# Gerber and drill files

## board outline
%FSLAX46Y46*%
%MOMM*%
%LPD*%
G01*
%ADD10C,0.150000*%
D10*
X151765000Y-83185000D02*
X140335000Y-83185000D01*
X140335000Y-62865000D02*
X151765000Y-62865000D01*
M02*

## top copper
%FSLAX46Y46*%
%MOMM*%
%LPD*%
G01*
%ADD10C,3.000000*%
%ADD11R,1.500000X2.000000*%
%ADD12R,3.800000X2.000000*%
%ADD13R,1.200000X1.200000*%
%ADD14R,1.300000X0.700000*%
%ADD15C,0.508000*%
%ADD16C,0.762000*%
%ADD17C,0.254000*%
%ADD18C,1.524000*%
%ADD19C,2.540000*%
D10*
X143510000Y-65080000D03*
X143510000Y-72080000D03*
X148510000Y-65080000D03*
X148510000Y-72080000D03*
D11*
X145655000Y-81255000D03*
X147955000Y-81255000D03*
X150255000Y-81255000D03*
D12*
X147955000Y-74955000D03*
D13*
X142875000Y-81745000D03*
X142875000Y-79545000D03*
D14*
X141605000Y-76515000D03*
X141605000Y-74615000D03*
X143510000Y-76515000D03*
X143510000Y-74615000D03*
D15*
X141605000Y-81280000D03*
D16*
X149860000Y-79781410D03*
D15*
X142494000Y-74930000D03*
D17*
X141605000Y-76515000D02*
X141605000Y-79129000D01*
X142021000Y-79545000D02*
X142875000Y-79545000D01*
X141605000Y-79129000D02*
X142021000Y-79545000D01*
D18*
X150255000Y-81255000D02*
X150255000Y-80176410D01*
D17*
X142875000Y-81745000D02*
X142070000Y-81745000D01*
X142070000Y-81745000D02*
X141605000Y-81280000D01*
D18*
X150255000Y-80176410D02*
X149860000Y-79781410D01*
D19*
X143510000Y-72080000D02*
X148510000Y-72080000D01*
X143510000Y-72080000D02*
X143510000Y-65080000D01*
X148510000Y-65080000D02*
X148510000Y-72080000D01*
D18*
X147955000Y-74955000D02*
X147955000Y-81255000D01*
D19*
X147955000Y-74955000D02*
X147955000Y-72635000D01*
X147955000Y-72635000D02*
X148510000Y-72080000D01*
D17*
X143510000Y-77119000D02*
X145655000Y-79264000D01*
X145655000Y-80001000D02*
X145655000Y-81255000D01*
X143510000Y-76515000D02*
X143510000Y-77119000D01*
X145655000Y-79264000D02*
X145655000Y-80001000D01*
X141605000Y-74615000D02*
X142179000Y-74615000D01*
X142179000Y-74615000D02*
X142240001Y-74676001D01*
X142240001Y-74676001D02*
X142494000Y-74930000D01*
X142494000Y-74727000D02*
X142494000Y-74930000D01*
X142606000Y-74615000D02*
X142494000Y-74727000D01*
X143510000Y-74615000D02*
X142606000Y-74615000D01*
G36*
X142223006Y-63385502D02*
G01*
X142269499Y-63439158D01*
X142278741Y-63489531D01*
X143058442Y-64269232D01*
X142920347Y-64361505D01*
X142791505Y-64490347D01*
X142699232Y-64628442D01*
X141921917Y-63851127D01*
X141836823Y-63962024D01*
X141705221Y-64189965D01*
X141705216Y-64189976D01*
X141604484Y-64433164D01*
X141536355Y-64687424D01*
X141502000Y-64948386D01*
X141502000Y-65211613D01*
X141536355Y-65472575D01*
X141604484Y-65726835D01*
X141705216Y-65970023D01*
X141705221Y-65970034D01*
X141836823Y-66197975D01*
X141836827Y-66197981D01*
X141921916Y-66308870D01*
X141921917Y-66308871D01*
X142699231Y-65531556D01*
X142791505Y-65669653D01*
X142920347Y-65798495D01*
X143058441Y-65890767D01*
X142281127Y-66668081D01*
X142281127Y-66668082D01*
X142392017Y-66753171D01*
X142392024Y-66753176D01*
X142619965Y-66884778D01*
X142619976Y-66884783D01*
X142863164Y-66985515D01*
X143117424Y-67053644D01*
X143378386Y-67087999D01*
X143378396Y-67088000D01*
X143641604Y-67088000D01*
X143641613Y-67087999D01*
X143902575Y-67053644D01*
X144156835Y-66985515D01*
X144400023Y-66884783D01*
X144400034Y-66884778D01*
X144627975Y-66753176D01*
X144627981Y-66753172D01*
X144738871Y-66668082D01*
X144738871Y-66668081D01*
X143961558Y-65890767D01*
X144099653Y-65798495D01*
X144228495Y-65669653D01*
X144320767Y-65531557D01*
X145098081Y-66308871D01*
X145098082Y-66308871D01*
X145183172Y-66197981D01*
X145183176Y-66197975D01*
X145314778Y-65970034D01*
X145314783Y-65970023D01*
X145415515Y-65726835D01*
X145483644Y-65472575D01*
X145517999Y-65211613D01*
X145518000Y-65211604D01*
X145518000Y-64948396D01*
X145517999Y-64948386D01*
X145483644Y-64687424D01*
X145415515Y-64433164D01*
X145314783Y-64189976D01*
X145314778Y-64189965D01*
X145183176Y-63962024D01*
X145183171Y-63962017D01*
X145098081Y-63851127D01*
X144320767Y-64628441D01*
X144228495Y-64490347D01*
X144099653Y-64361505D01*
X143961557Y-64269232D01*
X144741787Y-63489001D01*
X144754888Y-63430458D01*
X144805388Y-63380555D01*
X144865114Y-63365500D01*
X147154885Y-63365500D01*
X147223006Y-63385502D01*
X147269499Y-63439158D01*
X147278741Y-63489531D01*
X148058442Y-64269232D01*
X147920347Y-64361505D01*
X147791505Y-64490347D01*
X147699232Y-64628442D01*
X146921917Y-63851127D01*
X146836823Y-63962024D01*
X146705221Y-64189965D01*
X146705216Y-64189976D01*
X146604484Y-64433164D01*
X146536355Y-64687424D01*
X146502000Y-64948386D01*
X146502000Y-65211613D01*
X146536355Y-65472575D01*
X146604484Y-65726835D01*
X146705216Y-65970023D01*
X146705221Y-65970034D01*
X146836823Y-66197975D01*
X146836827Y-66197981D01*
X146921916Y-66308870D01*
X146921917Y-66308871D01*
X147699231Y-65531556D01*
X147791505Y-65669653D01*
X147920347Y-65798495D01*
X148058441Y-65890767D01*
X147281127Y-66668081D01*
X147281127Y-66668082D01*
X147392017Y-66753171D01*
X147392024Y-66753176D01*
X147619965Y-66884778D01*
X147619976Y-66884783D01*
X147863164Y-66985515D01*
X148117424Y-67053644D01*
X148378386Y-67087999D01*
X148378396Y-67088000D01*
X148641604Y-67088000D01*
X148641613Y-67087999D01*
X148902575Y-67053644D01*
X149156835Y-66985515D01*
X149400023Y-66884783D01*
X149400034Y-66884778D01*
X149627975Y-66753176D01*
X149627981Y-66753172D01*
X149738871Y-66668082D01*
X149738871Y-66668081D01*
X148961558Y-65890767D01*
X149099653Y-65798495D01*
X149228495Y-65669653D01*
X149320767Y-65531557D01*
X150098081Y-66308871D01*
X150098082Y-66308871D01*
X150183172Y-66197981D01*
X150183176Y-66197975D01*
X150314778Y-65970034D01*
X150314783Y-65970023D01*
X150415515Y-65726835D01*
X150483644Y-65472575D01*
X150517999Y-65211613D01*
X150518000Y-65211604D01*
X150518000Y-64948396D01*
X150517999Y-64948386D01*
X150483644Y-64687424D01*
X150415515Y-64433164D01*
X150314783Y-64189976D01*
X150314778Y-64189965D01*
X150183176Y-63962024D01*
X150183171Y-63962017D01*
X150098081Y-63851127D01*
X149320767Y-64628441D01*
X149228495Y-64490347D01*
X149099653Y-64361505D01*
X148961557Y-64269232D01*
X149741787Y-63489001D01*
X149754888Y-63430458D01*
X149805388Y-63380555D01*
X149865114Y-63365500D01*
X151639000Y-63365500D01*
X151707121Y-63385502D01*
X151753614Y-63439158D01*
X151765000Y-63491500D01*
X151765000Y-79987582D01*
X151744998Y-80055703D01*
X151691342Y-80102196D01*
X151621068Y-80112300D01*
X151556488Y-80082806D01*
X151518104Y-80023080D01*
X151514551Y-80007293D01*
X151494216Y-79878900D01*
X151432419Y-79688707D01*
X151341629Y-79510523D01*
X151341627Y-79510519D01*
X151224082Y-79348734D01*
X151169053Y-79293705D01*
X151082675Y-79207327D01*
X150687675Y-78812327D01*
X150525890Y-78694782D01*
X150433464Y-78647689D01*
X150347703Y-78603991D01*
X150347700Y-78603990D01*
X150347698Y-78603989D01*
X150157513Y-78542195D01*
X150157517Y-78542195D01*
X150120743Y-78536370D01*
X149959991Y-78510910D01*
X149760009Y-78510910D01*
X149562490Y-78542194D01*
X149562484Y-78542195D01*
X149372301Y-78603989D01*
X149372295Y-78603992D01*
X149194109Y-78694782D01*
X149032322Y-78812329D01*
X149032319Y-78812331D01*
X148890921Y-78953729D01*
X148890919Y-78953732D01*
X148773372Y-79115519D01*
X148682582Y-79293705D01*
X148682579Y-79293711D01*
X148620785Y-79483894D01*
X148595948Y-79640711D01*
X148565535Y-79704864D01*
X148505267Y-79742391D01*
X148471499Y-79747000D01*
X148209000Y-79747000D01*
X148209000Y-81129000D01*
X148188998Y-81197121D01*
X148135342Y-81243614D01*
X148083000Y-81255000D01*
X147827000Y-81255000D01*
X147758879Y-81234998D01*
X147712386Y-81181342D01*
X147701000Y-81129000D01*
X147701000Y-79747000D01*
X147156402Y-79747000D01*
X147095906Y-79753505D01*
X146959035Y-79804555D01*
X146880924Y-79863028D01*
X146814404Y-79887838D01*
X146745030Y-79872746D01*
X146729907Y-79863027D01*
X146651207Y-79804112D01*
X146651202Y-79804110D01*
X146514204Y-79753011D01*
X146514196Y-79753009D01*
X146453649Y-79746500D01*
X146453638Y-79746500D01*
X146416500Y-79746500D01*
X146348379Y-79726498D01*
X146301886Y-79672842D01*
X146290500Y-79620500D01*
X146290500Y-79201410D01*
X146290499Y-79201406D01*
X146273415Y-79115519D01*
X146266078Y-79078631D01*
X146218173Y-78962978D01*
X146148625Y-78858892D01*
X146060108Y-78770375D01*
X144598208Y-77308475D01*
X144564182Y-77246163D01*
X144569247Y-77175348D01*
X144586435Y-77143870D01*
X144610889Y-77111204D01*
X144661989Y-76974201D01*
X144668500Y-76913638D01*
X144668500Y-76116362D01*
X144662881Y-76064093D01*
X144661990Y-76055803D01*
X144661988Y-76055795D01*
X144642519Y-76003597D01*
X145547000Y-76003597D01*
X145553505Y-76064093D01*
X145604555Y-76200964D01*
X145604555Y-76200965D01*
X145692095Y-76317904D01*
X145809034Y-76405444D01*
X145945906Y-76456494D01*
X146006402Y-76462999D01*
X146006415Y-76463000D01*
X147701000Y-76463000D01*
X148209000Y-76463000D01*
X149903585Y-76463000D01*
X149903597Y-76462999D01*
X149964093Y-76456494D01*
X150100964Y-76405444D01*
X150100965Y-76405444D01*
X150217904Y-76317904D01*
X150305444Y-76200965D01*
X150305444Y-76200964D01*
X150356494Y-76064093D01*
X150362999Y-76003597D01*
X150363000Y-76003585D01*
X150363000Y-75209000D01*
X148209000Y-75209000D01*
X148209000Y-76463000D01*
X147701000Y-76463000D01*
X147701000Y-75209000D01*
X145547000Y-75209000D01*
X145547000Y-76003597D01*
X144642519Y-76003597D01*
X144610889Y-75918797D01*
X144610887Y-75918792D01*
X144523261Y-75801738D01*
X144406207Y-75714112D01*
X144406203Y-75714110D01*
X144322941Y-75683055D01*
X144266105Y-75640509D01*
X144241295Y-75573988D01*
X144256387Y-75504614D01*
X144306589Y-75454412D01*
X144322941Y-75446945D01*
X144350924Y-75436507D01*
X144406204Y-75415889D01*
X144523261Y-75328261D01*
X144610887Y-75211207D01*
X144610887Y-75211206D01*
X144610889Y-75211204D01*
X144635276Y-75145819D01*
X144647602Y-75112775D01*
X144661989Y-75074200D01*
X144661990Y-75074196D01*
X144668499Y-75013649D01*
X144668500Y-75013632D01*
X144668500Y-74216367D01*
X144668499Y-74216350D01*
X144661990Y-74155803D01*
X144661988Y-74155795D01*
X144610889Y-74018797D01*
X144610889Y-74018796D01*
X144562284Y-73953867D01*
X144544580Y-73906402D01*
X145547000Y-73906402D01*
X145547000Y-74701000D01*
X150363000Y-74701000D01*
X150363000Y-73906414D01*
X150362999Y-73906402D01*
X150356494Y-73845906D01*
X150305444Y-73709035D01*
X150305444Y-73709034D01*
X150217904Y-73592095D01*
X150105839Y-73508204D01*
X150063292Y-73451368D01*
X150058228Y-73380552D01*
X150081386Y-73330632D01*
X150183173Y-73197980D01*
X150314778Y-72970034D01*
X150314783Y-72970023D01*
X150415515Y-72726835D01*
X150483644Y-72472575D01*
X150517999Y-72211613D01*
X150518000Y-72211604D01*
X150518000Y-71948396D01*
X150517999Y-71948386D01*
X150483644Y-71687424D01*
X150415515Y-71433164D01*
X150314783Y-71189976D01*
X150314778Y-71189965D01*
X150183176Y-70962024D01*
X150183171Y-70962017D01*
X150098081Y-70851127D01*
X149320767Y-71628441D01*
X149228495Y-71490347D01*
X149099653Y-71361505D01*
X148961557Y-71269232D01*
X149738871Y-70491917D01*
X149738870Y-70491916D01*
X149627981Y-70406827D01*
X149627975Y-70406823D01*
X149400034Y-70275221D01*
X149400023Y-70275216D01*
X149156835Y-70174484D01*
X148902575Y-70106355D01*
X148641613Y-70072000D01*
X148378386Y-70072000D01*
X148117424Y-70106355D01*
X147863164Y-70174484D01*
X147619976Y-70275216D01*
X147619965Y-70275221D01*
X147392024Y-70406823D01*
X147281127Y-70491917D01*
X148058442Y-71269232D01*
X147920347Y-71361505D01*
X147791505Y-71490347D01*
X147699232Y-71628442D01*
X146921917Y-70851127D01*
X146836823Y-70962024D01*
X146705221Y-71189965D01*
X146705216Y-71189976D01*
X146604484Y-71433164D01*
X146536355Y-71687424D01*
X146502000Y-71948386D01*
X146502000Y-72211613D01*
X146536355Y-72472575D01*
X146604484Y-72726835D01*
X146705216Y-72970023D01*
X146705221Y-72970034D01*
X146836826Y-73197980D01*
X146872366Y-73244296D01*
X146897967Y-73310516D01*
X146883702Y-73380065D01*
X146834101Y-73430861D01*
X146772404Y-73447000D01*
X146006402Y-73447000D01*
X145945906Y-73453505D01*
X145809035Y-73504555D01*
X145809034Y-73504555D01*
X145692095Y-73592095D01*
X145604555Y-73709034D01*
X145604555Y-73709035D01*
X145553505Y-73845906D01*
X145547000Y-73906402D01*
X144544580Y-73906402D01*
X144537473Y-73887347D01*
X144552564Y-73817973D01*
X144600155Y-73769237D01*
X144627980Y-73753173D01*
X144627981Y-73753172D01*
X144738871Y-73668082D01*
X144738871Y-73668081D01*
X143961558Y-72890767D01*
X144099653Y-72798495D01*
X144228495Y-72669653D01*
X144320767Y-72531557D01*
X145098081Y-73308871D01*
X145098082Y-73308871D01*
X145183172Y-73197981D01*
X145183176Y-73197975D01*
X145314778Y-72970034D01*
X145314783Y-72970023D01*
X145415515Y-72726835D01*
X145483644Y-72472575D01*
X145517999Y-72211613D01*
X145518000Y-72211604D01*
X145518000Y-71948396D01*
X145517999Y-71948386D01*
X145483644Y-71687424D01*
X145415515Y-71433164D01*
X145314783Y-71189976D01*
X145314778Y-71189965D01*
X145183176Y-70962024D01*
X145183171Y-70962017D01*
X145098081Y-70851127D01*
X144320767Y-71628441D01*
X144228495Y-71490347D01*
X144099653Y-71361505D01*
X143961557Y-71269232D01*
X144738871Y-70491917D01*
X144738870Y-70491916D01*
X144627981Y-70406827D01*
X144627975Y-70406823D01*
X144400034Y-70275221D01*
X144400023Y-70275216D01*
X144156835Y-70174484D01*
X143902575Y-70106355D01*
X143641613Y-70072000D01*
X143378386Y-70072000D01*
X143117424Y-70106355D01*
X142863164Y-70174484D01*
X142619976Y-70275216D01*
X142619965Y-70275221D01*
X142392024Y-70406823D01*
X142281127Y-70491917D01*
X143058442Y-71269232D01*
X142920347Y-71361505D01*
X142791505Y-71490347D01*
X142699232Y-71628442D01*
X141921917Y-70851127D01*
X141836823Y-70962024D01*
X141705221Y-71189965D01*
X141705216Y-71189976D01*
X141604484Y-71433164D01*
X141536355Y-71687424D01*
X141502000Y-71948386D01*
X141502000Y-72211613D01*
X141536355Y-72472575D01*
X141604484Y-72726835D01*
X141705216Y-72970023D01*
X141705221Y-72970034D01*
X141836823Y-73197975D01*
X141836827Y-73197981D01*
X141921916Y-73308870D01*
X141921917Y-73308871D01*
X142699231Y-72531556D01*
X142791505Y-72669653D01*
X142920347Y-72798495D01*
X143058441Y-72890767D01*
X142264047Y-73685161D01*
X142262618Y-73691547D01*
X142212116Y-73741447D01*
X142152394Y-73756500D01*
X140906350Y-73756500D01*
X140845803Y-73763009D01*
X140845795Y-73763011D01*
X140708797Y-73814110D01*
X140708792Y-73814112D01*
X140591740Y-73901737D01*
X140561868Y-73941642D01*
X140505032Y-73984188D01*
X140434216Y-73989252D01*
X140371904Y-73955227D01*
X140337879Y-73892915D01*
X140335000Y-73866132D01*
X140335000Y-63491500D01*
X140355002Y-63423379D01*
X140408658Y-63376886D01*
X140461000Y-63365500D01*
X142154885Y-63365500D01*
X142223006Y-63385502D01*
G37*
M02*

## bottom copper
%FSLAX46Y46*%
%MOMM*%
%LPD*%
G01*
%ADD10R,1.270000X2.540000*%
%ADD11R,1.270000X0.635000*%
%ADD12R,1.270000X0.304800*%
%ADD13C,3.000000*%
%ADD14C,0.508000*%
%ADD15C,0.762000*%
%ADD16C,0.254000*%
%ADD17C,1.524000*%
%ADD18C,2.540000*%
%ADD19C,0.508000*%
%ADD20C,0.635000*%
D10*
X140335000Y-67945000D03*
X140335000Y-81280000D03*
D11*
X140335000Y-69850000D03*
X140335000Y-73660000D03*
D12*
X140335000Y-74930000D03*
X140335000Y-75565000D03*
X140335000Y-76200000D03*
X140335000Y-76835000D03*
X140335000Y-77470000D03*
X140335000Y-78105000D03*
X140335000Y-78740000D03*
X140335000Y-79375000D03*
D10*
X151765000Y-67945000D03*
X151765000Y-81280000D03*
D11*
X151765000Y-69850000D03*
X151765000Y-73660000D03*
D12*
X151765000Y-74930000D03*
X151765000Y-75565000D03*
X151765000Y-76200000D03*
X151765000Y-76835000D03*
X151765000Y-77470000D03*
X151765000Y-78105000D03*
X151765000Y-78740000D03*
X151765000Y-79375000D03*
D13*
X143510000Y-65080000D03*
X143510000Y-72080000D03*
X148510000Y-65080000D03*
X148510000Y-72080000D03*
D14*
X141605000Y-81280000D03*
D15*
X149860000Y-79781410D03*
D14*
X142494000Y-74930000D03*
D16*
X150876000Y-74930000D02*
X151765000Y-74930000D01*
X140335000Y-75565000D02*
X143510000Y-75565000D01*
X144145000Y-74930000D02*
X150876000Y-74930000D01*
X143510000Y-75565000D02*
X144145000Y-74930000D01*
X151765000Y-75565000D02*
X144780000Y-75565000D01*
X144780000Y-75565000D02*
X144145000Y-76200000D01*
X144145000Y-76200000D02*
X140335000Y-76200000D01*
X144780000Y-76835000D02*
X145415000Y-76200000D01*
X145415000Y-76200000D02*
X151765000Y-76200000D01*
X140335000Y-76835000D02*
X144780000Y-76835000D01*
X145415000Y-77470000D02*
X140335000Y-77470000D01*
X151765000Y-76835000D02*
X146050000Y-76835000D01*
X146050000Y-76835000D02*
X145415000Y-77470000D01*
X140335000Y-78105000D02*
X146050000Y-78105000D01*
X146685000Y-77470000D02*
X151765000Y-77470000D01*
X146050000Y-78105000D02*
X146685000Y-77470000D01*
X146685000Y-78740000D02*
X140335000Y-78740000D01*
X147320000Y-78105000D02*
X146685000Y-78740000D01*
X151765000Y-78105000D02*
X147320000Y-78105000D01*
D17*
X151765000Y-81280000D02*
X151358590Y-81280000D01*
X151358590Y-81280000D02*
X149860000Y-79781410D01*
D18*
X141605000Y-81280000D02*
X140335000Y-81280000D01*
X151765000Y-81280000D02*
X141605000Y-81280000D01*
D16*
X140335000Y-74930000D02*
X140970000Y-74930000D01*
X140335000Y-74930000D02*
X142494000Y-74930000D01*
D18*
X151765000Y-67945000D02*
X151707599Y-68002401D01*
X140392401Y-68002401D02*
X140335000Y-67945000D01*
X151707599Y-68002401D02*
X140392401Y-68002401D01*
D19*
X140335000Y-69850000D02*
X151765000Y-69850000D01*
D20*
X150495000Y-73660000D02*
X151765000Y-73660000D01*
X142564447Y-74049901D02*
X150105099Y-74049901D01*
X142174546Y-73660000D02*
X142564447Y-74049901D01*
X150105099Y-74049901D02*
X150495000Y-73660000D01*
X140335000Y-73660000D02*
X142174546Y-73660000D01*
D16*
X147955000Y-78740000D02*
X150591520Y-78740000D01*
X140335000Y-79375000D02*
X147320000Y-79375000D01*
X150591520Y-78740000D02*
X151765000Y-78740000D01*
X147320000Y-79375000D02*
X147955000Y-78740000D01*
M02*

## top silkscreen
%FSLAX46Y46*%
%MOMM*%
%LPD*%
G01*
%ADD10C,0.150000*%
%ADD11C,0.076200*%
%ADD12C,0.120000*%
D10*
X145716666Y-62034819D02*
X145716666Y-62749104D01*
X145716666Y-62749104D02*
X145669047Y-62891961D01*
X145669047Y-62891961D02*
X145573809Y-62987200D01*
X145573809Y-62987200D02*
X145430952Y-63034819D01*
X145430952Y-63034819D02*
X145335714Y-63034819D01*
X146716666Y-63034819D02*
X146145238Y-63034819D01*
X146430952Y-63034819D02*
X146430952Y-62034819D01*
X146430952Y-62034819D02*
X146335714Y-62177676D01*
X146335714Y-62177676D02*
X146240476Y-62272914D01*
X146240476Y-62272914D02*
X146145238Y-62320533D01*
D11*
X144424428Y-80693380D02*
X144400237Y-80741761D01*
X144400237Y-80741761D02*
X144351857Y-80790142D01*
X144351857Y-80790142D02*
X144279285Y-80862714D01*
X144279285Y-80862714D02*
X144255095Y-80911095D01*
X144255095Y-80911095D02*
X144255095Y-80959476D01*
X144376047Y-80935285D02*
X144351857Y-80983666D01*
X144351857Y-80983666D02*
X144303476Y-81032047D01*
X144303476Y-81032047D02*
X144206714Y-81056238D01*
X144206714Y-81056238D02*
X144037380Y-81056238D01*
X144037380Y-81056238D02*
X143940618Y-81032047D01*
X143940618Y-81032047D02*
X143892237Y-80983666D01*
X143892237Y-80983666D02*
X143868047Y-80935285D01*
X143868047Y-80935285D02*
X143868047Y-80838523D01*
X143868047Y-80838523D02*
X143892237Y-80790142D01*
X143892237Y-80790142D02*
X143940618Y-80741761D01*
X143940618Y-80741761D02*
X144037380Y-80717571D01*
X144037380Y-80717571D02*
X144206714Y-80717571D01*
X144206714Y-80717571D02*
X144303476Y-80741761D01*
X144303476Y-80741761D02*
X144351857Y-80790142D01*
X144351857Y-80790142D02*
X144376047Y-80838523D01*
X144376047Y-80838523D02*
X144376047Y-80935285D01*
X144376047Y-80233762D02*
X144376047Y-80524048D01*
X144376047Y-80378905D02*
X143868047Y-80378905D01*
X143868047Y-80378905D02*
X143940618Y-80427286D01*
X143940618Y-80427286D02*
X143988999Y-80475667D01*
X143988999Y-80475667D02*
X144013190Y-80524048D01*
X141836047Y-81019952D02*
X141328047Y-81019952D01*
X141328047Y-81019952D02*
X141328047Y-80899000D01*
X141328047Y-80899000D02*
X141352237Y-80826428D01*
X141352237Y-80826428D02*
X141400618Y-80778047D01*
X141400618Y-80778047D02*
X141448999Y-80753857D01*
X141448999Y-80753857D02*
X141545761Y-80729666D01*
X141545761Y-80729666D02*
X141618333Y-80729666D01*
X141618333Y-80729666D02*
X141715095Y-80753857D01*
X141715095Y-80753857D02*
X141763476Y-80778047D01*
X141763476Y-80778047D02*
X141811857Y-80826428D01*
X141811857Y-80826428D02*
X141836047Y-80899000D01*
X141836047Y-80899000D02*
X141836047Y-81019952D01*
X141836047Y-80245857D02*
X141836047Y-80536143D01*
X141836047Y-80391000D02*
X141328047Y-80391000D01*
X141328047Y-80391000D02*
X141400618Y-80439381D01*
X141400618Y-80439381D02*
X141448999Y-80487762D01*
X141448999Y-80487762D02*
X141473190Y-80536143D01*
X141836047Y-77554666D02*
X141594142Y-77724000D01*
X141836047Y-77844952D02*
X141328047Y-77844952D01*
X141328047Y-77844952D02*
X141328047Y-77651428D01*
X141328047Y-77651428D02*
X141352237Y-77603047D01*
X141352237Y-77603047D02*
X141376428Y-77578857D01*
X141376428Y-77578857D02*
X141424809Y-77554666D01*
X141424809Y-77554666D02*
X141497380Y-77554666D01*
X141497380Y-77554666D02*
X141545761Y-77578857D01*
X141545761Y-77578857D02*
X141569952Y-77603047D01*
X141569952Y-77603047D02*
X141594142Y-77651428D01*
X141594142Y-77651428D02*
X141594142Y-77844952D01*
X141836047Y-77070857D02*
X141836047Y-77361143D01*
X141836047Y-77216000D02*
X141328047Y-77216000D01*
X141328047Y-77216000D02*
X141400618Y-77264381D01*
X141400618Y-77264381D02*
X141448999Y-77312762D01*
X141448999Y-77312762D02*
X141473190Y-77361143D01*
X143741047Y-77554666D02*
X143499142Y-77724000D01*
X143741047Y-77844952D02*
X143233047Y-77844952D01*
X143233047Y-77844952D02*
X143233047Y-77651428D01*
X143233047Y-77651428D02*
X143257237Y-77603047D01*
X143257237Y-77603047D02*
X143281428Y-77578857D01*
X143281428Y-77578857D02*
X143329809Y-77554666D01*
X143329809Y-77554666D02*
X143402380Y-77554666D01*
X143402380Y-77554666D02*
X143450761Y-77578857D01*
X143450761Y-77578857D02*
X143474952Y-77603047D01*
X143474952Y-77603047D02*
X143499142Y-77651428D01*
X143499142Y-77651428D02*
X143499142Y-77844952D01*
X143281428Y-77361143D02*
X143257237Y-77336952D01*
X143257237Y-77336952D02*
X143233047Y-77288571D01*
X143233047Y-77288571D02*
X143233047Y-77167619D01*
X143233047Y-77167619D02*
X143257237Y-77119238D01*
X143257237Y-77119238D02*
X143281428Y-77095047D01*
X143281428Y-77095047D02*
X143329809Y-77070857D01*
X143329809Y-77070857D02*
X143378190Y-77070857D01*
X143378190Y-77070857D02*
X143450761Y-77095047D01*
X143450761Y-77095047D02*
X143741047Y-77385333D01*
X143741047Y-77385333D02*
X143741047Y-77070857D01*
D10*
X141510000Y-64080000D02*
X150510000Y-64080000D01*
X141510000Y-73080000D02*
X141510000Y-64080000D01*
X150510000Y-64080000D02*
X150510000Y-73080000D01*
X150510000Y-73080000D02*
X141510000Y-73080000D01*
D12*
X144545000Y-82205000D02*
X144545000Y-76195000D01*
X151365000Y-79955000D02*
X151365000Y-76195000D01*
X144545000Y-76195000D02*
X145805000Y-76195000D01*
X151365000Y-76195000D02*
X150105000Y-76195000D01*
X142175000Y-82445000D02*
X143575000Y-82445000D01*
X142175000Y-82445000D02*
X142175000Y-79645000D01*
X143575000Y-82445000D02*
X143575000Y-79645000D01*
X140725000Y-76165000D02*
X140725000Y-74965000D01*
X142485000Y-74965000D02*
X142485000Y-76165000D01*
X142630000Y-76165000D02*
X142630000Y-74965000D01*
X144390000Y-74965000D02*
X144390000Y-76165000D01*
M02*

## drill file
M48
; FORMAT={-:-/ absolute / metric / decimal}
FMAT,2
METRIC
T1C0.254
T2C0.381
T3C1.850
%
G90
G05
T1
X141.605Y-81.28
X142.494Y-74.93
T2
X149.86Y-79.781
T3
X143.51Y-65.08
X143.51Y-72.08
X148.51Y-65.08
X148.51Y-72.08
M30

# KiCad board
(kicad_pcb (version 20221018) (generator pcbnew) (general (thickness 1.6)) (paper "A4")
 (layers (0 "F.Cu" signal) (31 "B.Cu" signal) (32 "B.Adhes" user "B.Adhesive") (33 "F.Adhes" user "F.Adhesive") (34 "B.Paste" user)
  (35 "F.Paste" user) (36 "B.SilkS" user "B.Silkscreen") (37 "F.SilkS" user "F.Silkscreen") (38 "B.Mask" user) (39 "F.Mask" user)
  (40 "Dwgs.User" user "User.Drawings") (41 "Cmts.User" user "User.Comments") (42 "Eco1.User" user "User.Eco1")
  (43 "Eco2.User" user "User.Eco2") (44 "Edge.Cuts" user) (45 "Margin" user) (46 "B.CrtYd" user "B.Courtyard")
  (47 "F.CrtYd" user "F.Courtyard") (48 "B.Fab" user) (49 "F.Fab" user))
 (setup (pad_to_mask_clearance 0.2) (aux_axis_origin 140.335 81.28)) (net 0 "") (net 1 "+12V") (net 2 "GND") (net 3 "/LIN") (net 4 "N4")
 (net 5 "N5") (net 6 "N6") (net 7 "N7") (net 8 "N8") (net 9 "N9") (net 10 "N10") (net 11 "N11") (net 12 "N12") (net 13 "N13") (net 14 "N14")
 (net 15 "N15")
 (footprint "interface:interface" (layer "F.Cu") (at 140.335 63.5)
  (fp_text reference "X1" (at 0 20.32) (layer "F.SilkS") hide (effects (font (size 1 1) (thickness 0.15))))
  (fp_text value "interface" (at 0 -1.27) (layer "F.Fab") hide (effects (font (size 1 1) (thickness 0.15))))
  (pad "1" smd rect (at 0 4.445) (size 1.27 2.54) (layers "B.Cu") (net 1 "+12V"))
  (pad "2" smd rect (at 0 17.78) (size 1.27 2.54) (layers "B.Cu") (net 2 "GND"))
  (pad "3" smd rect (at 0 6.35) (size 1.27 0.635) (layers "B.Cu") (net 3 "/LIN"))
  (pad "4" smd rect (at 0 10.16) (size 1.27 0.635) (layers "B.Cu") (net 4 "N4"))
  (pad "5" smd rect (at 0 11.43) (size 1.27 0.3048) (layers "B.Cu") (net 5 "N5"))
  (pad "6" smd rect (at 0 12.065) (size 1.27 0.3048) (layers "B.Cu") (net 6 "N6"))
  (pad "7" smd rect (at 0 12.7) (size 1.27 0.3048) (layers "B.Cu") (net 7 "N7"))
  (pad "8" smd rect (at 0 13.335) (size 1.27 0.3048) (layers "B.Cu") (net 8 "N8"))
  (pad "9" smd rect (at 0 13.97) (size 1.27 0.3048) (layers "B.Cu") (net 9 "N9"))
  (pad "10" smd rect (at 0 14.605) (size 1.27 0.3048) (layers "B.Cu") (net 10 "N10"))
  (pad "11" smd rect (at 0 15.24) (size 1.27 0.3048) (layers "B.Cu") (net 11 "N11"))
  (pad "12" smd rect (at 0 15.875) (size 1.27 0.3048) (layers "B.Cu") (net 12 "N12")))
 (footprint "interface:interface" (layer "F.Cu") (at 151.765 63.5)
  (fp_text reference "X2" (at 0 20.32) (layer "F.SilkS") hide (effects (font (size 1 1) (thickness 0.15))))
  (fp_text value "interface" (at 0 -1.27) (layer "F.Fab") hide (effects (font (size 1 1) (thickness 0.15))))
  (pad "1" smd rect (at 0 4.445) (size 1.27 2.54) (layers "B.Cu") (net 1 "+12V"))
  (pad "2" smd rect (at 0 17.78) (size 1.27 2.54) (layers "B.Cu") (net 2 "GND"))
  (pad "3" smd rect (at 0 6.35) (size 1.27 0.635) (layers "B.Cu") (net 3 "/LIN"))
  (pad "4" smd rect (at 0 10.16) (size 1.27 0.635) (layers "B.Cu") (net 4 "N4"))
  (pad "5" smd rect (at 0 11.43) (size 1.27 0.3048) (layers "B.Cu") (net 6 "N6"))
  (pad "6" smd rect (at 0 12.065) (size 1.27 0.3048) (layers "B.Cu") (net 7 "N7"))
  (pad "7" smd rect (at 0 12.7) (size 1.27 0.3048) (layers "B.Cu") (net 8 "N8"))
  (pad "8" smd rect (at 0 13.335) (size 1.27 0.3048) (layers "B.Cu") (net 9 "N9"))
  (pad "9" smd rect (at 0 13.97) (size 1.27 0.3048) (layers "B.Cu") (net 10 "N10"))
  (pad "10" smd rect (at 0 14.605) (size 1.27 0.3048) (layers "B.Cu") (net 11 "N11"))
  (pad "11" smd rect (at 0 15.24) (size 1.27 0.3048) (layers "B.Cu") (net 12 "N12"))
  (pad "12" smd rect (at 0 15.875) (size 1.27 0.3048) (layers "B.Cu")))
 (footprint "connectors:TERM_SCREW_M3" (layer "F.Cu") (at 146.01 68.58)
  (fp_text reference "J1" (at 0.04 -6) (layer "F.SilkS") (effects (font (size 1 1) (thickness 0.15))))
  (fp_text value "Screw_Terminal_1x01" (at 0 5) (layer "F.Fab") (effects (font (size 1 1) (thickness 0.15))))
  (fp_line (start -4.5 -4.5) (end 4.5 -4.5) (stroke (width 0.15) (type solid)) (layer "F.SilkS"))
  (fp_line (start -4.5 4.5) (end -4.5 -4.5) (stroke (width 0.15) (type solid)) (layer "F.SilkS"))
  (fp_line (start 4.5 -4.5) (end 4.5 4.5) (stroke (width 0.15) (type solid)) (layer "F.SilkS"))
  (fp_line (start 4.5 4.5) (end -4.5 4.5) (stroke (width 0.15) (type solid)) (layer "F.SilkS"))
  (pad "1" thru_hole circle (at -2.5 -3.5) (size 3 3) (drill 1.85) (layers "*.Cu" "*.Mask") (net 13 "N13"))
  (pad "1" thru_hole circle (at -2.5 3.5) (size 3 3) (drill 1.85) (layers "*.Cu" "*.Mask") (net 13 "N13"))
  (pad "1" thru_hole circle (at 2.5 -3.5) (size 3 3) (drill 1.85) (layers "*.Cu" "*.Mask") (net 13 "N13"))
  (pad "1" thru_hole circle (at 2.5 3.5) (size 3 3) (drill 1.85) (layers "*.Cu" "*.Mask") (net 13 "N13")))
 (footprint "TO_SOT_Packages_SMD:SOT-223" (layer "F.Cu") (at 147.955 78.105 90)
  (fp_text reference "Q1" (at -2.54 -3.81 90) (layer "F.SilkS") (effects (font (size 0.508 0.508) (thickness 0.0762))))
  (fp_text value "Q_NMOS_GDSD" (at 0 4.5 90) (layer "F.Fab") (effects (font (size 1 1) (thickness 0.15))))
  (fp_line (start -4.1 -3.41) (end 1.91 -3.41) (stroke (width 0.12) (type solid)) (layer "F.SilkS"))
  (fp_line (start -1.85 3.41) (end 1.91 3.41) (stroke (width 0.12) (type solid)) (layer "F.SilkS"))
  (fp_line (start 1.91 -3.41) (end 1.91 -2.15) (stroke (width 0.12) (type solid)) (layer "F.SilkS"))
  (fp_line (start 1.91 3.41) (end 1.91 2.15) (stroke (width 0.12) (type solid)) (layer "F.SilkS"))
  (pad "1" smd rect (at -3.15 -2.3 90) (size 2 1.5) (layers "F.Cu" "F.Paste" "F.Mask") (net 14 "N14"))
  (pad "2" smd rect (at -3.15 0 90) (size 2 1.5) (layers "F.Cu" "F.Paste" "F.Mask") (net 13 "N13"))
  (pad "3" smd rect (at -3.15 2.3 90) (size 2 1.5) (layers "F.Cu" "F.Paste" "F.Mask") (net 2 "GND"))
  (pad "4" smd rect (at 3.15 0 90) (size 2 3.8) (layers "F.Cu" "F.Paste" "F.Mask") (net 13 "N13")))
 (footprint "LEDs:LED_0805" (layer "F.Cu") (at 142.875 80.645 90)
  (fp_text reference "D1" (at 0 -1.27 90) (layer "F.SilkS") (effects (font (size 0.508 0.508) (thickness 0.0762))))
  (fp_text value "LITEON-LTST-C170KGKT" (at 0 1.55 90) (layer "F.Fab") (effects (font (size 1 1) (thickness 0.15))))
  (fp_line (start -1.8 -0.7) (end -1.8 0.7) (stroke (width 0.12) (type solid)) (layer "F.SilkS"))
  (fp_line (start -1.8 -0.7) (end 1 -0.7) (stroke (width 0.12) (type solid)) (layer "F.SilkS"))
  (fp_line (start -1.8 0.7) (end 1 0.7) (stroke (width 0.12) (type solid)) (layer "F.SilkS"))
  (pad "1" smd rect (at -1.1 0 270) (size 1.2 1.2) (layers "F.Cu" "F.Paste" "F.Mask") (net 2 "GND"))
  (pad "2" smd rect (at 1.1 0 270) (size 1.2 1.2) (layers "F.Cu" "F.Paste" "F.Mask") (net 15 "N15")))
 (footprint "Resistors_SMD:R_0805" (layer "F.Cu") (at 141.605 75.565 90)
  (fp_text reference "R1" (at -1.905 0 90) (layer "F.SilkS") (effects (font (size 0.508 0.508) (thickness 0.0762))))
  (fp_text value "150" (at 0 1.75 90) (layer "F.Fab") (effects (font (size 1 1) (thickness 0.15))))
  (fp_line (start -0.6 -0.88) (end 0.6 -0.88) (stroke (width 0.12) (type solid)) (layer "F.SilkS"))
  (fp_line (start 0.6 0.88) (end -0.6 0.88) (stroke (width 0.12) (type solid)) (layer "F.SilkS"))
  (pad "1" smd rect (at -0.95 0 90) (size 0.7 1.3) (layers "F.Cu" "F.Paste" "F.Mask") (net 15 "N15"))
  (pad "2" smd rect (at 0.95 0 90) (size 0.7 1.3) (layers "F.Cu" "F.Paste" "F.Mask") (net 5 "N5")))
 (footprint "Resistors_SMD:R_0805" (layer "F.Cu") (at 143.51 75.565 90)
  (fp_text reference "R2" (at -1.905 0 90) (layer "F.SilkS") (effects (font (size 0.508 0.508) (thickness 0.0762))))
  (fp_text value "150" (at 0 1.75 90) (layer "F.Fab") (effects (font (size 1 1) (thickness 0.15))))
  (fp_line (start -0.6 -0.88) (end 0.6 -0.88) (stroke (width 0.12) (type solid)) (layer "F.SilkS"))
  (fp_line (start 0.6 0.88) (end -0.6 0.88) (stroke (width 0.12) (type solid)) (layer "F.SilkS"))
  (pad "1" smd rect (at -0.95 0 90) (size 0.7 1.3) (layers "F.Cu" "F.Paste" "F.Mask") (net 14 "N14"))
  (pad "2" smd rect (at 0.95 0 90) (size 0.7 1.3) (layers "F.Cu" "F.Paste" "F.Mask") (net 5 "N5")))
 (gr_line (start 151.765 83.185) (end 140.335 83.185) (stroke (width 0.15) (type solid)) (layer "Edge.Cuts"))
 (gr_line (start 140.335 62.865) (end 151.765 62.865) (stroke (width 0.15) (type solid)) (layer "Edge.Cuts"))
 (segment (start 150.876 74.93) (end 151.765 74.93) (width 0.254) (layer "B.Cu") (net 6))
 (segment (start 140.335 75.565) (end 143.51 75.565) (width 0.254) (layer "B.Cu") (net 6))
 (segment (start 144.145 74.93) (end 150.876 74.93) (width 0.254) (layer "B.Cu") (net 6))
 (segment (start 143.51 75.565) (end 144.145 74.93) (width 0.254) (layer "B.Cu") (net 6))
 (segment (start 151.765 75.565) (end 144.78 75.565) (width 0.254) (layer "B.Cu") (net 7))
 (segment (start 144.78 75.565) (end 144.145 76.2) (width 0.254) (layer "B.Cu") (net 7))
 (segment (start 144.145 76.2) (end 140.335 76.2) (width 0.254) (layer "B.Cu") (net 7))
 (segment (start 144.78 76.835) (end 145.415 76.2) (width 0.254) (layer "B.Cu") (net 8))
 (segment (start 145.415 76.2) (end 151.765 76.2) (width 0.254) (layer "B.Cu") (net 8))
 (segment (start 140.335 76.835) (end 144.78 76.835) (width 0.254) (layer "B.Cu") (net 8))
 (segment (start 145.415 77.47) (end 140.335 77.47) (width 0.254) (layer "B.Cu") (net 9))
 (segment (start 151.765 76.835) (end 146.05 76.835) (width 0.254) (layer "B.Cu") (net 9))
 (segment (start 146.05 76.835) (end 145.415 77.47) (width 0.254) (layer "B.Cu") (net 9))
 (segment (start 140.335 78.105) (end 146.05 78.105) (width 0.254) (layer "B.Cu") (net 10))
 (segment (start 146.685 77.47) (end 151.765 77.47) (width 0.254) (layer "B.Cu") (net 10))
 (segment (start 146.05 78.105) (end 146.685 77.47) (width 0.254) (layer "B.Cu") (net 10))
 (segment (start 146.685 78.74) (end 140.335 78.74) (width 0.254) (layer "B.Cu") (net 11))
 (segment (start 147.32 78.105) (end 146.685 78.74) (width 0.254) (layer "B.Cu") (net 11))
 (segment (start 151.765 78.105) (end 147.32 78.105) (width 0.254) (layer "B.Cu") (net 11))
 (segment (start 141.605 76.515) (end 141.605 79.129) (width 0.254) (layer "F.Cu") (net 15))
 (segment (start 142.021 79.545) (end 142.875 79.545) (width 0.254) (layer "F.Cu") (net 15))
 (segment (start 141.605 79.129) (end 142.021 79.545) (width 0.254) (layer "F.Cu") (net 15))
 (segment (start 150.255 81.255) (end 150.255 80.17641) (width 1.524) (layer "F.Cu") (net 2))
 (segment (start 142.875 81.745) (end 142.07 81.745) (width 0.254) (layer "F.Cu") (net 2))
 (segment (start 142.07 81.745) (end 141.605 81.28) (width 0.254) (layer "F.Cu") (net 2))
 (segment (start 150.255 80.17641) (end 149.86 79.78141) (width 1.524) (layer "F.Cu") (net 2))
 (via (at 141.605 81.28) (size 0.508) (drill 0.254) (layers "F.Cu" "B.Cu") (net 2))
 (via (at 149.86 79.78141) (size 0.762) (drill 0.381) (layers "F.Cu" "B.Cu") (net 2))
 (segment (start 151.765 81.28) (end 151.35859 81.28) (width 1.524) (layer "B.Cu") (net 2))
 (segment (start 151.35859 81.28) (end 149.86 79.78141) (width 1.524) (layer "B.Cu") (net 2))
 (segment (start 141.605 81.28) (end 140.335 81.28) (width 2.54) (layer "B.Cu") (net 2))
 (segment (start 151.765 81.28) (end 141.605 81.28) (width 2.54) (layer "B.Cu") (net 2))
 (segment (start 143.51 72.08) (end 148.51 72.08) (width 2.54) (layer "F.Cu") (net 13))
 (segment (start 143.51 72.08) (end 143.51 65.08) (width 2.54) (layer "F.Cu") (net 13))
 (segment (start 148.51 65.08) (end 148.51 72.08) (width 2.54) (layer "F.Cu") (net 13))
 (segment (start 147.955 74.955) (end 147.955 81.255) (width 1.524) (layer "F.Cu") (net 13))
 (segment (start 147.955 74.955) (end 147.955 72.635) (width 2.54) (layer "F.Cu") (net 13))
 (segment (start 147.955 72.635) (end 148.51 72.08) (width 2.54) (layer "F.Cu") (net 13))
 (segment (start 143.51 77.119) (end 145.655 79.264) (width 0.254) (layer "F.Cu") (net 14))
 (segment (start 145.655 80.001) (end 145.655 81.255) (width 0.254) (layer "F.Cu") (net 14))
 (segment (start 143.51 76.515) (end 143.51 77.119) (width 0.254) (layer "F.Cu") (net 14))
 (segment (start 145.655 79.264) (end 145.655 80.001) (width 0.254) (layer "F.Cu") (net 14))
 (segment (start 141.605 74.615) (end 142.179 74.615) (width 0.254) (layer "F.Cu") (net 5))
 (segment (start 142.179 74.615) (end 142.240001 74.676001) (width 0.254) (layer "F.Cu") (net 5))
 (segment (start 142.240001 74.676001) (end 142.494 74.93) (width 0.254) (layer "F.Cu") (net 5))
 (segment (start 142.494 74.727) (end 142.494 74.93) (width 0.254) (layer "F.Cu") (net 5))
 (segment (start 142.606 74.615) (end 142.494 74.727) (width 0.254) (layer "F.Cu") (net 5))
 (segment (start 143.51 74.615) (end 142.606 74.615) (width 0.254) (layer "F.Cu") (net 5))
 (via (at 142.494 74.93) (size 0.508) (drill 0.254) (layers "F.Cu" "B.Cu") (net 5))
 (segment (start 140.335 74.93) (end 140.97 74.93) (width 0.254) (layer "B.Cu") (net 5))
 (segment (start 140.335 74.93) (end 142.494 74.93) (width 0.254) (layer "B.Cu") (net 5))
 (segment (start 151.765 67.945) (end 151.707599 68.002401) (width 2.54) (layer "B.Cu") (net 1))
 (segment (start 140.392401 68.002401) (end 140.335 67.945) (width 2.54) (layer "B.Cu") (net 1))
 (segment (start 151.707599 68.002401) (end 140.392401 68.002401) (width 2.54) (layer "B.Cu") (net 1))
 (segment (start 140.335 69.85) (end 151.765 69.85) (width 0.508) (layer "B.Cu") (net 3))
 (segment (start 150.495 73.66) (end 151.765 73.66) (width 0.635) (layer "B.Cu") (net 4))
 (segment (start 142.564447 74.049901) (end 150.105099 74.049901) (width 0.635) (layer "B.Cu") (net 4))
 (segment (start 142.174546 73.66) (end 142.564447 74.049901) (width 0.635) (layer "B.Cu") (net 4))
 (segment (start 150.105099 74.049901) (end 150.495 73.66) (width 0.635) (layer "B.Cu") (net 4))
 (segment (start 140.335 73.66) (end 142.174546 73.66) (width 0.635) (layer "B.Cu") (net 4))
 (segment (start 147.955 78.74) (end 150.59152 78.74) (width 0.254) (layer "B.Cu") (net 12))
 (segment (start 140.335 79.375) (end 147.32 79.375) (width 0.254) (layer "B.Cu") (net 12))
 (segment (start 150.59152 78.74) (end 151.765 78.74) (width 0.254) (layer "B.Cu") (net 12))
 (segment (start 147.32 79.375) (end 147.955 78.74) (width 0.254) (layer "B.Cu") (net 12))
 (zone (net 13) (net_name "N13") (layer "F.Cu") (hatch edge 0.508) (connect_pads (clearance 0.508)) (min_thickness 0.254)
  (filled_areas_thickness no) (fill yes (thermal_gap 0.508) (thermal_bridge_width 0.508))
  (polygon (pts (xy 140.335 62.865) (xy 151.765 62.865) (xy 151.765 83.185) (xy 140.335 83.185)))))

